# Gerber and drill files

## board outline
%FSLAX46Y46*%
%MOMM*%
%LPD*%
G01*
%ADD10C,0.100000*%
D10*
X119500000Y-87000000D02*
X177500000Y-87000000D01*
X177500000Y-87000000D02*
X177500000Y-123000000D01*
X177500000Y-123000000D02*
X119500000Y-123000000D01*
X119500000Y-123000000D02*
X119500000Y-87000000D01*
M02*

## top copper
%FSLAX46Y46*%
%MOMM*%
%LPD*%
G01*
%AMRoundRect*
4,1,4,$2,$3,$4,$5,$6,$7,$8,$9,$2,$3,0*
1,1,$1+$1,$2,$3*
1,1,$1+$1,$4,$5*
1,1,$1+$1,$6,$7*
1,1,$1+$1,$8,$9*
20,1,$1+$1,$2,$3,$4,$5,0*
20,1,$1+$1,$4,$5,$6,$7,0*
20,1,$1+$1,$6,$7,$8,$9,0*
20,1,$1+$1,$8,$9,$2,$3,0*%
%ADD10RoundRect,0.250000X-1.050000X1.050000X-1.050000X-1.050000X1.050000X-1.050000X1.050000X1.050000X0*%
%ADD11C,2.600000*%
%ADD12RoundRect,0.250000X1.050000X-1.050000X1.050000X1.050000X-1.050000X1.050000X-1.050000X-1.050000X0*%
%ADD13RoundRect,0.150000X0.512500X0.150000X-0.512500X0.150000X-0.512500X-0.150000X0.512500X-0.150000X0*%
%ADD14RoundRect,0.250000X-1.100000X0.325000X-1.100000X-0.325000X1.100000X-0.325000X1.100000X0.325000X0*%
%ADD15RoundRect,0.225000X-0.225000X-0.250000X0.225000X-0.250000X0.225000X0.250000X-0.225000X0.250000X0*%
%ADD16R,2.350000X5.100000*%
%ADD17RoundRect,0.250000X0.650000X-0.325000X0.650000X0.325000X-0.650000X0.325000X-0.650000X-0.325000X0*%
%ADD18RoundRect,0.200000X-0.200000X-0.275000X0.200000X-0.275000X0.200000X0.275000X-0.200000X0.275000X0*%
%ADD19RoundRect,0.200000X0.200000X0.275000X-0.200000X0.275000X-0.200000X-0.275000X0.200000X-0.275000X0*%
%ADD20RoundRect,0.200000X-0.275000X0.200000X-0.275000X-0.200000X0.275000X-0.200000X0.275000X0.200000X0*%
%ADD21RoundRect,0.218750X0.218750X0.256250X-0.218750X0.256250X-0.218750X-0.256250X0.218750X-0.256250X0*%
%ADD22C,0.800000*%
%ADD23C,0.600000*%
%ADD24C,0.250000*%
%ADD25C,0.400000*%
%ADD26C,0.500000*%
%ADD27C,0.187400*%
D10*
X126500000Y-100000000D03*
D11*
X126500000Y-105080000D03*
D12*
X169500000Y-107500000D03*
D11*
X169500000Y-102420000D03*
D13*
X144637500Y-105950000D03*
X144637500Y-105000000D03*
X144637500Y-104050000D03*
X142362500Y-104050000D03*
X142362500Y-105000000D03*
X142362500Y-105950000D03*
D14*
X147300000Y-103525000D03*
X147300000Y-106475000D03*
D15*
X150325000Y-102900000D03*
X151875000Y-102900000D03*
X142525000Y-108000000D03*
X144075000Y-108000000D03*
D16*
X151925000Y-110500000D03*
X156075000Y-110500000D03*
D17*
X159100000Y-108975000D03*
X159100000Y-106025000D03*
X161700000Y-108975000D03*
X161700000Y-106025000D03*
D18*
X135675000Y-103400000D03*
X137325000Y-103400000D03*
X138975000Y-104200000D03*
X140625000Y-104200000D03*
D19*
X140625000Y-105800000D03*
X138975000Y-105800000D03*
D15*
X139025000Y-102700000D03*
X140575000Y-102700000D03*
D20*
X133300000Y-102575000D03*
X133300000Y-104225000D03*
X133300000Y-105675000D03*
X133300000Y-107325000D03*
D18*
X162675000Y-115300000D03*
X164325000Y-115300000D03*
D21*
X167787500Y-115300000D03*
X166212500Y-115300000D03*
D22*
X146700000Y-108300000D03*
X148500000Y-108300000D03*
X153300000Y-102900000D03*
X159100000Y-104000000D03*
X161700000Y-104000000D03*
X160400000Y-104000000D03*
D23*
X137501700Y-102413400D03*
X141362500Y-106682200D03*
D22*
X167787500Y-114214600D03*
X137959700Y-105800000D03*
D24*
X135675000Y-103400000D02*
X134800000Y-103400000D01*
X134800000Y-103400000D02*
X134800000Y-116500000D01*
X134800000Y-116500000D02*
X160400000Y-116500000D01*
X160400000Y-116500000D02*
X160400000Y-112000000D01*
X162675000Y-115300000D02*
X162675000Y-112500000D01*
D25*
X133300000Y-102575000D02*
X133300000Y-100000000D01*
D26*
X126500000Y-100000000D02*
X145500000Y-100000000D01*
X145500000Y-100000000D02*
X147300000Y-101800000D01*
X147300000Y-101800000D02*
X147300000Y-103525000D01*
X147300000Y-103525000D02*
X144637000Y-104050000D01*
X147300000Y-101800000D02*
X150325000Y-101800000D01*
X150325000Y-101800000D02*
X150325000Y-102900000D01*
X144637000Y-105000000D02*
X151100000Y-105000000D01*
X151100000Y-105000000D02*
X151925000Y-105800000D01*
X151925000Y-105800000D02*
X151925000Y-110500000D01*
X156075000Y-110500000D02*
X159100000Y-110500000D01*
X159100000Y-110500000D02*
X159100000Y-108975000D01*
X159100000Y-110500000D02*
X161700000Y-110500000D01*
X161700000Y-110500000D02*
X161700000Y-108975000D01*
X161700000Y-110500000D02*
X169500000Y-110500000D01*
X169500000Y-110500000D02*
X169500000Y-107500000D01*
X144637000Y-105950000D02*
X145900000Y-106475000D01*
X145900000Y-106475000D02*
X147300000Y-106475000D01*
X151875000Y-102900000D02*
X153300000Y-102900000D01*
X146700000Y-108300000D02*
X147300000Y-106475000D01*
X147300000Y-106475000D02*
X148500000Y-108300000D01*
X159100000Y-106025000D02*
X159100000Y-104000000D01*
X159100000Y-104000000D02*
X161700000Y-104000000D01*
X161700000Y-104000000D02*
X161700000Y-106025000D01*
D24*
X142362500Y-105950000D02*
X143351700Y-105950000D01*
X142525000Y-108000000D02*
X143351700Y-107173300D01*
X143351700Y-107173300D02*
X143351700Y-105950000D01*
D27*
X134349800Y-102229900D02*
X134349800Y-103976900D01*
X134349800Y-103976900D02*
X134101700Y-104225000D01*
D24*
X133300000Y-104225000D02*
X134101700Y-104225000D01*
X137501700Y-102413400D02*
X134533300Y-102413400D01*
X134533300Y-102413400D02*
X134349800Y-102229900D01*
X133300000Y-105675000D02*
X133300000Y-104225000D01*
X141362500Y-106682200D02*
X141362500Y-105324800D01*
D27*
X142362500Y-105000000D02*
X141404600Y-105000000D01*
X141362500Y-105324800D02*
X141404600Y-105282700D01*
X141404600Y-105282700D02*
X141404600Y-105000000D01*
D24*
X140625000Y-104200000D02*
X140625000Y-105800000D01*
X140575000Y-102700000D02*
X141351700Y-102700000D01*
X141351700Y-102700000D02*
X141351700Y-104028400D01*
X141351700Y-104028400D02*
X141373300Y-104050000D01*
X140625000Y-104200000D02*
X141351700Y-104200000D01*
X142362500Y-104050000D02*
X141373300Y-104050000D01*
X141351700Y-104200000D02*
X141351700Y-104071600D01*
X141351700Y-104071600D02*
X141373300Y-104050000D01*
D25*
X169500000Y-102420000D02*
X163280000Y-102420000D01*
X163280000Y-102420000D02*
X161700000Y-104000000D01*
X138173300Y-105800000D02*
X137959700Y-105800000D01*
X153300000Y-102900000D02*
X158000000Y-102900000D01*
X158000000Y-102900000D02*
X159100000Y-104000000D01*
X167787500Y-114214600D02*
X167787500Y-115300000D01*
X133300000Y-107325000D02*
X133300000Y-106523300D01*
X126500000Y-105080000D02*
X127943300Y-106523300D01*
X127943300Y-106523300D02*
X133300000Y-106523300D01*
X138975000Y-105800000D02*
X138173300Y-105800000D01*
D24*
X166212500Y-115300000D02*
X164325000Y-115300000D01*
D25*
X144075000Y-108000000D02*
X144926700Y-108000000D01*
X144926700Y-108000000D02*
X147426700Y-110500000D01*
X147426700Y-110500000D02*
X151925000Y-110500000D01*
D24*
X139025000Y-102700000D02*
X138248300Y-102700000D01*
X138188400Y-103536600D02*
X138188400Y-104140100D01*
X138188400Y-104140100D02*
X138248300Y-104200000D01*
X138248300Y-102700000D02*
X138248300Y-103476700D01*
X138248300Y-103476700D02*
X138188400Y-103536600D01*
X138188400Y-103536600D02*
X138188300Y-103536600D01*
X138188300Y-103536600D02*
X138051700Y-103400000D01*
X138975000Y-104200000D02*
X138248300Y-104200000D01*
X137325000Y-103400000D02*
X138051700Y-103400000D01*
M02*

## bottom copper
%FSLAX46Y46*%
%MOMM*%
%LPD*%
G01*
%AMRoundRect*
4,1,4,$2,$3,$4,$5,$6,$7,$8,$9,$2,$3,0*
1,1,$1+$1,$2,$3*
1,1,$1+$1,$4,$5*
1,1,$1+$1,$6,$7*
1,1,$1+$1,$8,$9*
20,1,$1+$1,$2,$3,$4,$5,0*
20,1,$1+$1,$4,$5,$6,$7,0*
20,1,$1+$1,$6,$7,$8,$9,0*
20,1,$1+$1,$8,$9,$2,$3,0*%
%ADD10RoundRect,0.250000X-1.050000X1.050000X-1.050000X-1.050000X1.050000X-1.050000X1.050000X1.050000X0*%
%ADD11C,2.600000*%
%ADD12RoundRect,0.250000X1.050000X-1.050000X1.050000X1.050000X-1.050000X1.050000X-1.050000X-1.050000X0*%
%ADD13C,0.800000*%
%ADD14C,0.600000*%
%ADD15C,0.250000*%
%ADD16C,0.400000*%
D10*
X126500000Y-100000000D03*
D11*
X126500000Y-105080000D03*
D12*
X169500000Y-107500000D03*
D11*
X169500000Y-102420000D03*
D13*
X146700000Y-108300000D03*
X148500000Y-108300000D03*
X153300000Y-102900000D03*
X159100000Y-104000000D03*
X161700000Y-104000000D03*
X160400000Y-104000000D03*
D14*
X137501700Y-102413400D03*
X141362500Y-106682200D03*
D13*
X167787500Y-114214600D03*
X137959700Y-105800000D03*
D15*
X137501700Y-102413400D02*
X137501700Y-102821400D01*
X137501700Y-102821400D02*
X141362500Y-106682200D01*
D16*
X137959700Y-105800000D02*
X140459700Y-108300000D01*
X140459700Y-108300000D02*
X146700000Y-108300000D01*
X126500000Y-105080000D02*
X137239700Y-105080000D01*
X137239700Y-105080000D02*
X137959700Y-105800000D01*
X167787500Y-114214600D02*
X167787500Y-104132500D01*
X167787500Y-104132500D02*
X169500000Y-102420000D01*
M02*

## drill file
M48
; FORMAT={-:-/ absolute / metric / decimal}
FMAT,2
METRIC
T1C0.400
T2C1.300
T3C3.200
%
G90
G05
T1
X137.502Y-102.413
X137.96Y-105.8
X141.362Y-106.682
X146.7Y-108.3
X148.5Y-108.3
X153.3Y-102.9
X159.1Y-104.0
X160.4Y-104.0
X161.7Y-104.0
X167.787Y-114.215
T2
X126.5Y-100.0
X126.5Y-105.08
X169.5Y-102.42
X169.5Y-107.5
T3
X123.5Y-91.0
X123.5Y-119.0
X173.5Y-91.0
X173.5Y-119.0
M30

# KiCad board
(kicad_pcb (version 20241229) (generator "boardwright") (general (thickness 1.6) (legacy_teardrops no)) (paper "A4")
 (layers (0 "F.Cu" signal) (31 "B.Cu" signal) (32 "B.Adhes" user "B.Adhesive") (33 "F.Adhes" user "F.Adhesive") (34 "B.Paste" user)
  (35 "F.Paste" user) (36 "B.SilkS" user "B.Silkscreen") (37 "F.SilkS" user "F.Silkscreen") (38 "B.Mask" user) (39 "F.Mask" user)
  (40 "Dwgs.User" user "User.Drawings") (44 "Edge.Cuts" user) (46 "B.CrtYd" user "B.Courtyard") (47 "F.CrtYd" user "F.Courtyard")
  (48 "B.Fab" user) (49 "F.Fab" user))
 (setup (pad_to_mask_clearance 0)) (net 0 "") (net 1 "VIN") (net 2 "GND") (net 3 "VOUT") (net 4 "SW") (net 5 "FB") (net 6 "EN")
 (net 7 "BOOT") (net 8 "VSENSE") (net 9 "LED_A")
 (gr_line (start 119.5 87) (end 177.5 87) (stroke (width 0.1) (type default)) (layer "Edge.Cuts"))
 (gr_line (start 177.5 87) (end 177.5 123) (stroke (width 0.1) (type default)) (layer "Edge.Cuts"))
 (gr_line (start 177.5 123) (end 119.5 123) (stroke (width 0.1) (type default)) (layer "Edge.Cuts"))
 (gr_line (start 119.5 123) (end 119.5 87) (stroke (width 0.1) (type default)) (layer "Edge.Cuts"))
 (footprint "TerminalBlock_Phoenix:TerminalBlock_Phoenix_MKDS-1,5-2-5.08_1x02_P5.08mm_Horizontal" (layer "F.Cu") (at 126.5 100 -90)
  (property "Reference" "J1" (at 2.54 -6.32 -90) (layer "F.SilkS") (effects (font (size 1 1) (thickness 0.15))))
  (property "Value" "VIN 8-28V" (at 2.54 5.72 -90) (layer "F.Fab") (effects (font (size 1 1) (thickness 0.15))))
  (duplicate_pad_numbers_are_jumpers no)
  (pad "1" thru_hole roundrect (at 0 0 -90) (size 2.6 2.6) (drill 1.3) (layers "*.Cu" "*.Mask") (remove_unused_layers no)
   (roundrect_rratio 0.096154) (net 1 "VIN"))
  (pad "2" thru_hole circle (at 5.08 0 -90) (size 2.6 2.6) (drill 1.3) (layers "*.Cu" "*.Mask") (remove_unused_layers no) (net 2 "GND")))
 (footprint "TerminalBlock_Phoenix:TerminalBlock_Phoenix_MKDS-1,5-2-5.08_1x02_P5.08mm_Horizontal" (layer "F.Cu") (at 169.5 107.5 90)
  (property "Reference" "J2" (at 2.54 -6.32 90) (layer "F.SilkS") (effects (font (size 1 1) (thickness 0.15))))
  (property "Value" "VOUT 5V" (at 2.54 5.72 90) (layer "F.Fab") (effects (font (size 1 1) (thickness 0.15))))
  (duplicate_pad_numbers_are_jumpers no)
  (pad "1" thru_hole roundrect (at 0 0 90) (size 2.6 2.6) (drill 1.3) (layers "*.Cu" "*.Mask") (remove_unused_layers no)
   (roundrect_rratio 0.096154) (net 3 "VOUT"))
  (pad "2" thru_hole circle (at 5.08 0 90) (size 2.6 2.6) (drill 1.3) (layers "*.Cu" "*.Mask") (remove_unused_layers no) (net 2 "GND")))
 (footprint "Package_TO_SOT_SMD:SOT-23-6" (layer "F.Cu") (at 143.5 105 180)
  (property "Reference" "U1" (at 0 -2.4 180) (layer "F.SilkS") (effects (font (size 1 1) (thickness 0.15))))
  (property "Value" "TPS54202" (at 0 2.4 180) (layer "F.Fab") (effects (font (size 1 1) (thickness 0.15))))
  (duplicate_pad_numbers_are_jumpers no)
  (pad "1" smd roundrect (at -1.1375 -0.95 180) (size 1.325 0.6) (layers "F.Cu" "F.Mask" "F.Paste") (roundrect_rratio 0.25) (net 2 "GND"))
  (pad "2" smd roundrect (at -1.1375 0 180) (size 1.325 0.6) (layers "F.Cu" "F.Mask" "F.Paste") (roundrect_rratio 0.25) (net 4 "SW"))
  (pad "3" smd roundrect (at -1.1375 0.95 180) (size 1.325 0.6) (layers "F.Cu" "F.Mask" "F.Paste") (roundrect_rratio 0.25) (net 1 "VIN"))
  (pad "4" smd roundrect (at 1.1375 0.95 180) (size 1.325 0.6) (layers "F.Cu" "F.Mask" "F.Paste") (roundrect_rratio 0.25) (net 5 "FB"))
  (pad "5" smd roundrect (at 1.1375 0 180) (size 1.325 0.6) (layers "F.Cu" "F.Mask" "F.Paste") (roundrect_rratio 0.25) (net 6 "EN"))
  (pad "6" smd roundrect (at 1.1375 -0.95 180) (size 1.325 0.6) (layers "F.Cu" "F.Mask" "F.Paste") (roundrect_rratio 0.25) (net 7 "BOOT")))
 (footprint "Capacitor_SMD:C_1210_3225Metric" (layer "F.Cu") (at 147.3 105 -90)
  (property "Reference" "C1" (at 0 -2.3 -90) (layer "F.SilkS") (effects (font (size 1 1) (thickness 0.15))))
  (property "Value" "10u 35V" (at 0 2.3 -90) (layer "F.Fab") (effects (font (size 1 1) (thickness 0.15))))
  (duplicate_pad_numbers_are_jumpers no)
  (pad "1" smd roundrect (at -1.475 0 -90) (size 1.15 2.7) (layers "F.Cu" "F.Mask" "F.Paste") (roundrect_rratio 0.217391) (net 1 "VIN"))
  (pad "2" smd roundrect (at 1.475 0 -90) (size 1.15 2.7) (layers "F.Cu" "F.Mask" "F.Paste") (roundrect_rratio 0.217391) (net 2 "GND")))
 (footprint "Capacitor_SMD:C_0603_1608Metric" (layer "F.Cu") (at 151.1 102.9)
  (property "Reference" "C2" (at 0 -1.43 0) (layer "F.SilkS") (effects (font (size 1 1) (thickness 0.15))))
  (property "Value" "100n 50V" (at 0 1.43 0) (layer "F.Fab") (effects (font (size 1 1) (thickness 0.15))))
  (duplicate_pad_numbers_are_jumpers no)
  (pad "1" smd roundrect (at -0.775 0) (size 0.9 0.95) (layers "F.Cu" "F.Mask" "F.Paste") (roundrect_rratio 0.25) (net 1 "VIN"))
  (pad "2" smd roundrect (at 0.775 0) (size 0.9 0.95) (layers "F.Cu" "F.Mask" "F.Paste") (roundrect_rratio 0.25) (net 2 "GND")))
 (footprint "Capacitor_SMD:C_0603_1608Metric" (layer "F.Cu") (at 143.3 108)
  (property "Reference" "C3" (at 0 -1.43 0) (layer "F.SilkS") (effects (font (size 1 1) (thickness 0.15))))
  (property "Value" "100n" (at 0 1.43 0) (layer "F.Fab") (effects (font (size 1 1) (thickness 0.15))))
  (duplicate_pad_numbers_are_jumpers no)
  (pad "1" smd roundrect (at -0.775 0) (size 0.9 0.95) (layers "F.Cu" "F.Mask" "F.Paste") (roundrect_rratio 0.25) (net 7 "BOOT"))
  (pad "2" smd roundrect (at 0.775 0) (size 0.9 0.95) (layers "F.Cu" "F.Mask" "F.Paste") (roundrect_rratio 0.25) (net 4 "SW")))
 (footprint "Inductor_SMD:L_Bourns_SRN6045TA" (layer "F.Cu") (at 154 110.5)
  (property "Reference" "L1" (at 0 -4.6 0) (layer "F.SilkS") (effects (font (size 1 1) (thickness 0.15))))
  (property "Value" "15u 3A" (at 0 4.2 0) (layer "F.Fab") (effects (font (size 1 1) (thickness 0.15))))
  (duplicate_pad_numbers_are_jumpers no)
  (pad "1" smd rect (at -2.075 0) (size 2.35 5.1) (layers "F.Cu" "F.Mask" "F.Paste") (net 4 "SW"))
  (pad "2" smd rect (at 2.075 0) (size 2.35 5.1) (layers "F.Cu" "F.Mask" "F.Paste") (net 3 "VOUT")))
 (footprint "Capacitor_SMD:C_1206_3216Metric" (layer "F.Cu") (at 159.1 107.5 90)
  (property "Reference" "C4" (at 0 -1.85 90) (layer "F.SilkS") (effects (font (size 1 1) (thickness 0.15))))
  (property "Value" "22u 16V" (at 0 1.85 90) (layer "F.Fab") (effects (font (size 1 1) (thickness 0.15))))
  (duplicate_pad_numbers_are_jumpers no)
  (pad "1" smd roundrect (at -1.475 0 90) (size 1.15 1.8) (layers "F.Cu" "F.Mask" "F.Paste") (roundrect_rratio 0.217391) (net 3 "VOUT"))
  (pad "2" smd roundrect (at 1.475 0 90) (size 1.15 1.8) (layers "F.Cu" "F.Mask" "F.Paste") (roundrect_rratio 0.217391) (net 2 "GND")))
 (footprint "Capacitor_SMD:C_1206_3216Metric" (layer "F.Cu") (at 161.7 107.5 90)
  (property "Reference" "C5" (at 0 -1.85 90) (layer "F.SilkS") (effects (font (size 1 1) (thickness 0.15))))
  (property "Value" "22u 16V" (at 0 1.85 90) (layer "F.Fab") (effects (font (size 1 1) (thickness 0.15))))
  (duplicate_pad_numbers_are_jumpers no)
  (pad "1" smd roundrect (at -1.475 0 90) (size 1.15 1.8) (layers "F.Cu" "F.Mask" "F.Paste") (roundrect_rratio 0.217391) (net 3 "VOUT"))
  (pad "2" smd roundrect (at 1.475 0 90) (size 1.15 1.8) (layers "F.Cu" "F.Mask" "F.Paste") (roundrect_rratio 0.217391) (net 2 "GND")))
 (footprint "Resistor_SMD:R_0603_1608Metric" (layer "F.Cu") (at 136.5 103.4)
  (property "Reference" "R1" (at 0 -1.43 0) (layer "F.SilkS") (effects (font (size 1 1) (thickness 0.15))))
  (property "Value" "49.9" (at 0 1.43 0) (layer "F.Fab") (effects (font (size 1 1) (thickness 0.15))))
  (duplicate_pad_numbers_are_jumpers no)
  (pad "1" smd roundrect (at -0.825 0) (size 0.8 0.95) (layers "F.Cu" "F.Mask" "F.Paste") (roundrect_rratio 0.25) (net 3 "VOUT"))
  (pad "2" smd roundrect (at 0.825 0) (size 0.8 0.95) (layers "F.Cu" "F.Mask" "F.Paste") (roundrect_rratio 0.25) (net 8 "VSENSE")))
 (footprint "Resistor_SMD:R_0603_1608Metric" (layer "F.Cu") (at 139.8 104.2)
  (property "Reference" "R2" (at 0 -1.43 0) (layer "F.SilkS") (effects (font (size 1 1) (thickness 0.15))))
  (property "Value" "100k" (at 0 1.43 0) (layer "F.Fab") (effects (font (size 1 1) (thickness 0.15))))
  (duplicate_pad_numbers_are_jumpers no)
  (pad "1" smd roundrect (at -0.825 0) (size 0.8 0.95) (layers "F.Cu" "F.Mask" "F.Paste") (roundrect_rratio 0.25) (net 8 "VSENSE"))
  (pad "2" smd roundrect (at 0.825 0) (size 0.8 0.95) (layers "F.Cu" "F.Mask" "F.Paste") (roundrect_rratio 0.25) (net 5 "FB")))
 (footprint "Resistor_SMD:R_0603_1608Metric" (layer "F.Cu") (at 139.8 105.8 180)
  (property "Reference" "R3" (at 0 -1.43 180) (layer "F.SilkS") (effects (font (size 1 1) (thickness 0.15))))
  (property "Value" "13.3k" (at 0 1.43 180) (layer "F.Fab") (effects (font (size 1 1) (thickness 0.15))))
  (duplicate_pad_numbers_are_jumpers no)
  (pad "1" smd roundrect (at -0.825 0 180) (size 0.8 0.95) (layers "F.Cu" "F.Mask" "F.Paste") (roundrect_rratio 0.25) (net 5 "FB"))
  (pad "2" smd roundrect (at 0.825 0 180) (size 0.8 0.95) (layers "F.Cu" "F.Mask" "F.Paste") (roundrect_rratio 0.25) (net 2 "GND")))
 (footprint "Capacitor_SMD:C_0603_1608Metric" (layer "F.Cu") (at 139.8 102.7)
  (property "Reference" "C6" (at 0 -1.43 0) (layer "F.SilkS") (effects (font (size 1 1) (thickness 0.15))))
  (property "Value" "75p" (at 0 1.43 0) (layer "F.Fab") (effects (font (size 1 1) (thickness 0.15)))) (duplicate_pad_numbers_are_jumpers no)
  (pad "1" smd roundrect (at -0.775 0) (size 0.9 0.95) (layers "F.Cu" "F.Mask" "F.Paste") (roundrect_rratio 0.25) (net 8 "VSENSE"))
  (pad "2" smd roundrect (at 0.775 0) (size 0.9 0.95) (layers "F.Cu" "F.Mask" "F.Paste") (roundrect_rratio 0.25) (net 5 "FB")))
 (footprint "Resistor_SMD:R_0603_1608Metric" (layer "F.Cu") (at 133.3 103.4 -90)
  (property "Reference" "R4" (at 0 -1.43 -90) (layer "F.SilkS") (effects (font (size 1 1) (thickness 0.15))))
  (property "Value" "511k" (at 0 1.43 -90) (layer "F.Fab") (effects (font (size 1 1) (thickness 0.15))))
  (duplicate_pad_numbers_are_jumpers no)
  (pad "1" smd roundrect (at -0.825 0 -90) (size 0.8 0.95) (layers "F.Cu" "F.Mask" "F.Paste") (roundrect_rratio 0.25) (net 1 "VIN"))
  (pad "2" smd roundrect (at 0.825 0 -90) (size 0.8 0.95) (layers "F.Cu" "F.Mask" "F.Paste") (roundrect_rratio 0.25) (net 6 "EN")))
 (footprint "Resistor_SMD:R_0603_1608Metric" (layer "F.Cu") (at 133.3 106.5 -90)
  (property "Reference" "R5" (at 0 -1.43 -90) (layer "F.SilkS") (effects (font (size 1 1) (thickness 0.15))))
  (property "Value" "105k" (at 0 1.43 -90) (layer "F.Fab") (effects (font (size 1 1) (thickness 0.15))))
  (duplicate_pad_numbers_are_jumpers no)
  (pad "1" smd roundrect (at -0.825 0 -90) (size 0.8 0.95) (layers "F.Cu" "F.Mask" "F.Paste") (roundrect_rratio 0.25) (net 6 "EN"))
  (pad "2" smd roundrect (at 0.825 0 -90) (size 0.8 0.95) (layers "F.Cu" "F.Mask" "F.Paste") (roundrect_rratio 0.25) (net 2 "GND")))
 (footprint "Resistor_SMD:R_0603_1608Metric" (layer "F.Cu") (at 163.5 115.3)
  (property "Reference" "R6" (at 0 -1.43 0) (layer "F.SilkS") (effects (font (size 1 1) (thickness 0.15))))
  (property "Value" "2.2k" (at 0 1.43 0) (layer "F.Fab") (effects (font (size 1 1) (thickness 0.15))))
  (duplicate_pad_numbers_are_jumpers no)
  (pad "1" smd roundrect (at -0.825 0) (size 0.8 0.95) (layers "F.Cu" "F.Mask" "F.Paste") (roundrect_rratio 0.25) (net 3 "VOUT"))
  (pad "2" smd roundrect (at 0.825 0) (size 0.8 0.95) (layers "F.Cu" "F.Mask" "F.Paste") (roundrect_rratio 0.25) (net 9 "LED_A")))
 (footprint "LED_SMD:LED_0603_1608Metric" (layer "F.Cu") (at 167 115.3 180)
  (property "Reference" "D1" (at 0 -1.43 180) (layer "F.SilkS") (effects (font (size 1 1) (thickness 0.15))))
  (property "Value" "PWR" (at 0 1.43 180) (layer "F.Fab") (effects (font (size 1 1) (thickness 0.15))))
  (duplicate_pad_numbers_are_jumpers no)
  (pad "1" smd roundrect (at -0.7875 0 180) (size 0.875 0.95) (layers "F.Cu" "F.Mask" "F.Paste") (roundrect_rratio 0.25) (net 2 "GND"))
  (pad "2" smd roundrect (at 0.7875 0 180) (size 0.875 0.95) (layers "F.Cu" "F.Mask" "F.Paste") (roundrect_rratio 0.25) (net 9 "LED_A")))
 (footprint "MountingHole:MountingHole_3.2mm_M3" (layer "F.Cu") (at 123.5 91)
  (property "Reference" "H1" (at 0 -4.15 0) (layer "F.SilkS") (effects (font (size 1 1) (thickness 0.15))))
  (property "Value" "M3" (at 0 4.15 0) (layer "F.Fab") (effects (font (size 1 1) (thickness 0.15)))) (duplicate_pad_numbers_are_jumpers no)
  (pad "" np_thru_hole circle (at 0 0) (size 3.2 3.2) (drill 3.2) (layers "*.Cu" "*.Mask")))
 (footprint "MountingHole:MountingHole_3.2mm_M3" (layer "F.Cu") (at 173.5 91)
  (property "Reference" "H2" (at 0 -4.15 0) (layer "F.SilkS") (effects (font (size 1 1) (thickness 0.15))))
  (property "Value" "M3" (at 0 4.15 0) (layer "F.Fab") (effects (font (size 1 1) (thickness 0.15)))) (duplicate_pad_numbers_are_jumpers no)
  (pad "" np_thru_hole circle (at 0 0) (size 3.2 3.2) (drill 3.2) (layers "*.Cu" "*.Mask")))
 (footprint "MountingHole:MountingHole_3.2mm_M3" (layer "F.Cu") (at 123.5 119)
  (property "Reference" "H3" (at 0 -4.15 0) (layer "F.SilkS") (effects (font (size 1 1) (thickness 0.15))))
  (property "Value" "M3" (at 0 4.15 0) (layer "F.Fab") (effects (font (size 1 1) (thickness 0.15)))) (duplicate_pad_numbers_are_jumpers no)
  (pad "" np_thru_hole circle (at 0 0) (size 3.2 3.2) (drill 3.2) (layers "*.Cu" "*.Mask")))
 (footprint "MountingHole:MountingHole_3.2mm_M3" (layer "F.Cu") (at 173.5 119)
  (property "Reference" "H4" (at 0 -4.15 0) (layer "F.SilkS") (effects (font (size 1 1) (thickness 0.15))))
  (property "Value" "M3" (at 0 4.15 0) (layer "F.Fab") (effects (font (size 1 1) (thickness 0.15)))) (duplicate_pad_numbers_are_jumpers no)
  (pad "" np_thru_hole circle (at 0 0) (size 3.2 3.2) (drill 3.2) (layers "*.Cu" "*.Mask")))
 (via (at 146.7 108.3) (size 0.8) (drill 0.4) (layers "F.Cu" "B.Cu") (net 2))
 (via (at 148.5 108.3) (size 0.8) (drill 0.4) (layers "F.Cu" "B.Cu") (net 2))
 (via (at 153.3 102.9) (size 0.8) (drill 0.4) (layers "F.Cu" "B.Cu") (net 2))
 (via (at 159.1 104.0) (size 0.8) (drill 0.4) (layers "F.Cu" "B.Cu") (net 2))
 (via (at 161.7 104.0) (size 0.8) (drill 0.4) (layers "F.Cu" "B.Cu") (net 2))
 (via (at 160.4 104.0) (size 0.8) (drill 0.4) (layers "F.Cu" "B.Cu") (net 2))
 (segment (start 135.675 103.4) (end 134.8 103.4) (width 0.25) (layer "F.Cu") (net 3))
 (segment (start 134.8 103.4) (end 134.8 116.5) (width 0.25) (layer "F.Cu") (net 3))
 (segment (start 134.8 116.5) (end 160.4 116.5) (width 0.25) (layer "F.Cu") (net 3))
 (segment (start 160.4 116.5) (end 160.4 112.0) (width 0.25) (layer "F.Cu") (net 3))
 (segment (start 162.675 115.3) (end 162.675 112.5) (width 0.25) (layer "F.Cu") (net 3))
 (segment (start 133.3 102.575) (end 133.3 100.0) (width 0.4) (layer "F.Cu") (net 1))
 (segment (start 126.5 100.0) (end 145.5 100.0) (width 0.5) (layer "F.Cu") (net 1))
 (segment (start 145.5 100.0) (end 147.3 101.8) (width 0.5) (layer "F.Cu") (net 1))
 (segment (start 147.3 101.8) (end 147.3 103.525) (width 0.5) (layer "F.Cu") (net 1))
 (segment (start 147.3 103.525) (end 144.637 104.05) (width 0.5) (layer "F.Cu") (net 1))
 (segment (start 147.3 101.8) (end 150.325 101.8) (width 0.5) (layer "F.Cu") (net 1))
 (segment (start 150.325 101.8) (end 150.325 102.9) (width 0.5) (layer "F.Cu") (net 1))
 (segment (start 144.637 105.0) (end 151.1 105.0) (width 0.5) (layer "F.Cu") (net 4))
 (segment (start 151.1 105.0) (end 151.925 105.8) (width 0.5) (layer "F.Cu") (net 4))
 (segment (start 151.925 105.8) (end 151.925 110.5) (width 0.5) (layer "F.Cu") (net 4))
 (segment (start 156.075 110.5) (end 159.1 110.5) (width 0.5) (layer "F.Cu") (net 3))
 (segment (start 159.1 110.5) (end 159.1 108.975) (width 0.5) (layer "F.Cu") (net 3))
 (segment (start 159.1 110.5) (end 161.7 110.5) (width 0.5) (layer "F.Cu") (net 3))
 (segment (start 161.7 110.5) (end 161.7 108.975) (width 0.5) (layer "F.Cu") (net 3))
 (segment (start 161.7 110.5) (end 169.5 110.5) (width 0.5) (layer "F.Cu") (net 3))
 (segment (start 169.5 110.5) (end 169.5 107.5) (width 0.5) (layer "F.Cu") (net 3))
 (segment (start 144.637 105.95) (end 145.9 106.475) (width 0.5) (layer "F.Cu") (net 2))
 (segment (start 145.9 106.475) (end 147.3 106.475) (width 0.5) (layer "F.Cu") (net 2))
 (segment (start 151.875 102.9) (end 153.3 102.9) (width 0.5) (layer "F.Cu") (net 2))
 (segment (start 146.7 108.3) (end 147.3 106.475) (width 0.5) (layer "F.Cu") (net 2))
 (segment (start 147.3 106.475) (end 148.5 108.3) (width 0.5) (layer "F.Cu") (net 2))
 (segment (start 159.1 106.025) (end 159.1 104.0) (width 0.5) (layer "F.Cu") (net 2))
 (segment (start 159.1 104.0) (end 161.7 104.0) (width 0.5) (layer "F.Cu") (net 2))
 (segment (start 161.7 104.0) (end 161.7 106.025) (width 0.5) (layer "F.Cu") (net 2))
 (segment (start 142.3625 105.95) (end 143.3517 105.95) (width 0.25) (layer "F.Cu") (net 7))
 (segment (start 142.525 108) (end 143.3517 107.1733) (width 0.25) (layer "F.Cu") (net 7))
 (segment (start 143.3517 107.1733) (end 143.3517 105.95) (width 0.25) (layer "F.Cu") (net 7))
 (segment (start 137.5017 102.4134) (end 137.5017 102.8214) (width 0.25) (layer "B.Cu") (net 6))
 (segment (start 137.5017 102.8214) (end 141.3625 106.6822) (width 0.25) (layer "B.Cu") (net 6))
 (segment (start 134.3498 102.2299) (end 134.3498 103.9769) (width 0.1874) (layer "F.Cu") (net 6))
 (segment (start 134.3498 103.9769) (end 134.1017 104.225) (width 0.1874) (layer "F.Cu") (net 6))
 (segment (start 133.3 104.225) (end 134.1017 104.225) (width 0.25) (layer "F.Cu") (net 6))
 (segment (start 137.5017 102.4134) (end 134.5333 102.4134) (width 0.25) (layer "F.Cu") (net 6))
 (segment (start 134.5333 102.4134) (end 134.3498 102.2299) (width 0.25) (layer "F.Cu") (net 6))
 (segment (start 133.3 105.675) (end 133.3 104.225) (width 0.25) (layer "F.Cu") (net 6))
 (segment (start 141.3625 106.6822) (end 141.3625 105.3248) (width 0.25) (layer "F.Cu") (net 6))
 (segment (start 142.3625 105) (end 141.4046 105) (width 0.1874) (layer "F.Cu") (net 6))
 (segment (start 141.3625 105.3248) (end 141.4046 105.2827) (width 0.1874) (layer "F.Cu") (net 6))
 (segment (start 141.4046 105.2827) (end 141.4046 105) (width 0.1874) (layer "F.Cu") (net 6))
 (segment (start 140.625 104.2) (end 140.625 105.8) (width 0.25) (layer "F.Cu") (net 5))
 (segment (start 140.575 102.7) (end 141.3517 102.7) (width 0.25) (layer "F.Cu") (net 5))
 (segment (start 141.3517 102.7) (end 141.3517 104.0284) (width 0.25) (layer "F.Cu") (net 5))
 (segment (start 141.3517 104.0284) (end 141.3733 104.05) (width 0.25) (layer "F.Cu") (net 5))
 (segment (start 140.625 104.2) (end 141.3517 104.2) (width 0.25) (layer "F.Cu") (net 5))
 (segment (start 142.3625 104.05) (end 141.3733 104.05) (width 0.25) (layer "F.Cu") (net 5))
 (segment (start 141.3517 104.2) (end 141.3517 104.0716) (width 0.25) (layer "F.Cu") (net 5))
 (segment (start 141.3517 104.0716) (end 141.3733 104.05) (width 0.25) (layer "F.Cu") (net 5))
 (segment (start 169.5 102.42) (end 163.28 102.42) (width 0.4) (layer "F.Cu") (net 2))
 (segment (start 163.28 102.42) (end 161.7 104) (width 0.4) (layer "F.Cu") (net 2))
 (segment (start 137.9597 105.8) (end 140.4597 108.3) (width 0.4) (layer "B.Cu") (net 2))
 (segment (start 140.4597 108.3) (end 146.7 108.3) (width 0.4) (layer "B.Cu") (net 2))
 (segment (start 138.1733 105.8) (end 137.9597 105.8) (width 0.4) (layer "F.Cu") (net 2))
 (segment (start 126.5 105.08) (end 137.2397 105.08) (width 0.4) (layer "B.Cu") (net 2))
 (segment (start 137.2397 105.08) (end 137.9597 105.8) (width 0.4) (layer "B.Cu") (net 2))
 (segment (start 167.7875 114.2146) (end 167.7875 104.1325) (width 0.4) (layer "B.Cu") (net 2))
 (segment (start 167.7875 104.1325) (end 169.5 102.42) (width 0.4) (layer "B.Cu") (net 2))
 (segment (start 153.3 102.9) (end 158 102.9) (width 0.4) (layer "F.Cu") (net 2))
 (segment (start 158 102.9) (end 159.1 104) (width 0.4) (layer "F.Cu") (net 2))
 (segment (start 167.7875 114.2146) (end 167.7875 115.3) (width 0.4) (layer "F.Cu") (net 2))
 (segment (start 133.3 107.325) (end 133.3 106.5233) (width 0.4) (layer "F.Cu") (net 2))
 (segment (start 126.5 105.08) (end 127.9433 106.5233) (width 0.4) (layer "F.Cu") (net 2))
 (segment (start 127.9433 106.5233) (end 133.3 106.5233) (width 0.4) (layer "F.Cu") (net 2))
 (segment (start 138.975 105.8) (end 138.1733 105.8) (width 0.4) (layer "F.Cu") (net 2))
 (segment (start 166.2125 115.3) (end 164.325 115.3) (width 0.25) (layer "F.Cu") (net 9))
 (segment (start 144.075 108) (end 144.9267 108) (width 0.4) (layer "F.Cu") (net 4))
 (segment (start 144.9267 108) (end 147.4267 110.5) (width 0.4) (layer "F.Cu") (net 4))
 (segment (start 147.4267 110.5) (end 151.925 110.5) (width 0.4) (layer "F.Cu") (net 4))
 (segment (start 139.025 102.7) (end 138.2483 102.7) (width 0.25) (layer "F.Cu") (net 8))
 (segment (start 138.1884 103.5366) (end 138.1884 104.1401) (width 0.25) (layer "F.Cu") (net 8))
 (segment (start 138.1884 104.1401) (end 138.2483 104.2) (width 0.25) (layer "F.Cu") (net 8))
 (segment (start 138.2483 102.7) (end 138.2483 103.4767) (width 0.25) (layer "F.Cu") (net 8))
 (segment (start 138.2483 103.4767) (end 138.1884 103.5366) (width 0.25) (layer "F.Cu") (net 8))
 (segment (start 138.1884 103.5366) (end 138.1883 103.5366) (width 0.25) (layer "F.Cu") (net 8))
 (segment (start 138.1883 103.5366) (end 138.0517 103.4) (width 0.25) (layer "F.Cu") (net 8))
 (segment (start 138.975 104.2) (end 138.2483 104.2) (width 0.25) (layer "F.Cu") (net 8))
 (segment (start 137.325 103.4) (end 138.0517 103.4) (width 0.25) (layer "F.Cu") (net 8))
 (via (at 137.5017 102.4134) (size 0.6) (drill 0.4) (layers "F.Cu" "B.Cu") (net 6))
 (via (at 141.3625 106.6822) (size 0.6) (drill 0.4) (layers "F.Cu" "B.Cu") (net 6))
 (via (at 167.7875 114.2146) (size 0.8) (drill 0.4) (layers "F.Cu" "B.Cu") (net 2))
 (via (at 137.9597 105.8) (size 0.8) (drill 0.4) (layers "F.Cu" "B.Cu") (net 2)))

